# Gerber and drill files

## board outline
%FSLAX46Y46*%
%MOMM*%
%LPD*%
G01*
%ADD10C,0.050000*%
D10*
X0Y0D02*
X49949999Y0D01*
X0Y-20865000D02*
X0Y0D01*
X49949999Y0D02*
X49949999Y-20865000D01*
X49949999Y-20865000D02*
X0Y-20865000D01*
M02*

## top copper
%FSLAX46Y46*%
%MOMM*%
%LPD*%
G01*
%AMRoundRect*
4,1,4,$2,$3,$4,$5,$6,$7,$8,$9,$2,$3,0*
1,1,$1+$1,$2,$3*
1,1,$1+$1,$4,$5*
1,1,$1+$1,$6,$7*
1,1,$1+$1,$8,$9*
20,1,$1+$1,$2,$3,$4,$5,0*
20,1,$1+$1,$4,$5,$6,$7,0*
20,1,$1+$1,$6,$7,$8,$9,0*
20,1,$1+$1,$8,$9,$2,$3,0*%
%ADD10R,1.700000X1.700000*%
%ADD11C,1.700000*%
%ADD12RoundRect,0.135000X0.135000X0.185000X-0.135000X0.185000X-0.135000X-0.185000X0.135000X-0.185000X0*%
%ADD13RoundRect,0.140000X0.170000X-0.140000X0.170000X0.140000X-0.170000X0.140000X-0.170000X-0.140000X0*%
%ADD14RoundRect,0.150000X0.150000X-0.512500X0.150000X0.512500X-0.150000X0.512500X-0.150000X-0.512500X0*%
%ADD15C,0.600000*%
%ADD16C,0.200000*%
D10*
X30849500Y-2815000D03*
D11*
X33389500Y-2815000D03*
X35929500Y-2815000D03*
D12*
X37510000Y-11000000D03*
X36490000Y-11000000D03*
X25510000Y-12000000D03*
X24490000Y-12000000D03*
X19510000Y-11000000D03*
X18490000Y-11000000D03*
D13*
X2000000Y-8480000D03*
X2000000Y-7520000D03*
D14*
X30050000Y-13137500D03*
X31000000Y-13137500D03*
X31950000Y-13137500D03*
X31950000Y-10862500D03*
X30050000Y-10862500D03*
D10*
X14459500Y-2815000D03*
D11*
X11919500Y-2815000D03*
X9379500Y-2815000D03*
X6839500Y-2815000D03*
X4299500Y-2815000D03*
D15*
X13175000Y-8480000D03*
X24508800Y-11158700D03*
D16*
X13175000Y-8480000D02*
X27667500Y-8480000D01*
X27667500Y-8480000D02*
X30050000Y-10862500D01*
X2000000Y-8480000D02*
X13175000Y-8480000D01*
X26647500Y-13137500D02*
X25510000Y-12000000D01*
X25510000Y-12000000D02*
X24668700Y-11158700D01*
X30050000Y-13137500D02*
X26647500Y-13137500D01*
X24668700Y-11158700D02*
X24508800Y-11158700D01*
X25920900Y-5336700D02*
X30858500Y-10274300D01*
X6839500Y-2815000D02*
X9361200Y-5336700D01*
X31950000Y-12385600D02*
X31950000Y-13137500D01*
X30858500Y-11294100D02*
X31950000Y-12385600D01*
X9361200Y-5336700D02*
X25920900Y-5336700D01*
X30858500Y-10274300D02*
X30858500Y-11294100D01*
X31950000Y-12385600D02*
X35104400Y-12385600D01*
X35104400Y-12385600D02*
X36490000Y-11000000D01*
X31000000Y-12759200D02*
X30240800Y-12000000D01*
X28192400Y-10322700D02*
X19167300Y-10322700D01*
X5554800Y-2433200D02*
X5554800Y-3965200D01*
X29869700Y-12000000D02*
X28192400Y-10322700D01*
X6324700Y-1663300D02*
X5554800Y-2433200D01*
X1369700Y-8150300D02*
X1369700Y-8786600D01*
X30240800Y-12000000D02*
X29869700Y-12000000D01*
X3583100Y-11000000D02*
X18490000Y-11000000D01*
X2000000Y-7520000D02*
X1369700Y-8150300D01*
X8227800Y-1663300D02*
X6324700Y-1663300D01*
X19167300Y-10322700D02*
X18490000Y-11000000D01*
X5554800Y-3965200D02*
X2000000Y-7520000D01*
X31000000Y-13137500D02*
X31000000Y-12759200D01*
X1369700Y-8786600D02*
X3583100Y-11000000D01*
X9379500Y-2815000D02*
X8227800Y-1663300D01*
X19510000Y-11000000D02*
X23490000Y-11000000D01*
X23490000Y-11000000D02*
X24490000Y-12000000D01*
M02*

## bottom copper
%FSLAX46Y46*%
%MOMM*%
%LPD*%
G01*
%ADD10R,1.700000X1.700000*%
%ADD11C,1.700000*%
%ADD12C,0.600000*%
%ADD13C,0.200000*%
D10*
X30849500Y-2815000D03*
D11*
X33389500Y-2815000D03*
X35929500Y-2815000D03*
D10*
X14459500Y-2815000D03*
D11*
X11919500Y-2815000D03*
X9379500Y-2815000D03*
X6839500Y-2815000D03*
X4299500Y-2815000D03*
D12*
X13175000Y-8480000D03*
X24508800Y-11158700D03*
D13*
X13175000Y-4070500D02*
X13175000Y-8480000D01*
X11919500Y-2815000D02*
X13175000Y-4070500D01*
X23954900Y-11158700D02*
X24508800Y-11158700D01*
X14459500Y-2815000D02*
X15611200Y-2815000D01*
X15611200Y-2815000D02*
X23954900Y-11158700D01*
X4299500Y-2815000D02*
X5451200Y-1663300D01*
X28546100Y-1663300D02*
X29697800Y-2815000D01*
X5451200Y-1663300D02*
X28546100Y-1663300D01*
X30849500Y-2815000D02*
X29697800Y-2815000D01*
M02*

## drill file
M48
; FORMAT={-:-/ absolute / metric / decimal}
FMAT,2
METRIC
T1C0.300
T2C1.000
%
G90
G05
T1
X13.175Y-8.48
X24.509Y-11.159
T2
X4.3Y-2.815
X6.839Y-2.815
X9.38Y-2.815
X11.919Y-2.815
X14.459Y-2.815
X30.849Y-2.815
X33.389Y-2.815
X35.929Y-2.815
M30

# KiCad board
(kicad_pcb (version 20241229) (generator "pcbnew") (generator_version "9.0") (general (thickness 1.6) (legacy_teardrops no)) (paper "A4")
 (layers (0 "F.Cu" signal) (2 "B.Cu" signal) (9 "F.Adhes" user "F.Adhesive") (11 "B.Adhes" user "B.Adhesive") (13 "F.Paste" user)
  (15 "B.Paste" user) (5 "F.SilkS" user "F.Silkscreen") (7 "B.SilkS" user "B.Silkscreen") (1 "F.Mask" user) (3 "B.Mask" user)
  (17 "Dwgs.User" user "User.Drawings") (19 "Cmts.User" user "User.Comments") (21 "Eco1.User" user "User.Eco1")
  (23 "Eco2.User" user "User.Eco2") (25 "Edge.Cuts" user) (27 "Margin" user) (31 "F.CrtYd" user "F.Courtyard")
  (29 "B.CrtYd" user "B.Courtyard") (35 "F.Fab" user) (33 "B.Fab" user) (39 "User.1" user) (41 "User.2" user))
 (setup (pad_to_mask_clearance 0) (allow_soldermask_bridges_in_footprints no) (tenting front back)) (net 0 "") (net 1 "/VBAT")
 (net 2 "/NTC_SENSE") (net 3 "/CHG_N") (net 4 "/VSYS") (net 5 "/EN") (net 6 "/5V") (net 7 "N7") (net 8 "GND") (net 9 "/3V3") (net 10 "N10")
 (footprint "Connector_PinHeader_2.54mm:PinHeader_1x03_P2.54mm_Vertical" (layer "F.Cu") (at 30.8495 2.815 90)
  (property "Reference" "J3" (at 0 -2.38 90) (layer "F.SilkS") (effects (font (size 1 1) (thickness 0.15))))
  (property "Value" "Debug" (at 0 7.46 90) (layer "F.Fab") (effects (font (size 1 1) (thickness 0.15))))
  (pad "1" thru_hole rect (at 0 0 90) (size 1.7 1.7) (drill 1) (layers "*.Cu" "*.Mask") (remove_unused_layers no) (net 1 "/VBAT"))
  (pad "2" thru_hole circle (at 0 2.54 90) (size 1.7 1.7) (drill 1) (layers "*.Cu" "*.Mask") (remove_unused_layers no) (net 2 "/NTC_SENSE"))
  (pad "3" thru_hole circle (at 0 5.08 90) (size 1.7 1.7) (drill 1) (layers "*.Cu" "*.Mask") (remove_unused_layers no) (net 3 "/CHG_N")))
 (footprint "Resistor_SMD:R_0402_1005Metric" (layer "F.Cu") (at 37 11 180)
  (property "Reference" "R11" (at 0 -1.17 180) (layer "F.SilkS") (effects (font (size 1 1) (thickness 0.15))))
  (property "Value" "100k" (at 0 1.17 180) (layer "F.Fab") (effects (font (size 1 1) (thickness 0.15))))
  (pad "1" smd roundrect (at -0.51 0 180) (size 0.54 0.64) (layers "F.Cu" "F.Mask" "F.Paste") (roundrect_rratio 0.25) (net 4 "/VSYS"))
  (pad "2" smd roundrect (at 0.51 0 180) (size 0.54 0.64) (layers "F.Cu" "F.Mask" "F.Paste") (roundrect_rratio 0.25) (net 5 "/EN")))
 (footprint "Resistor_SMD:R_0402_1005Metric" (layer "F.Cu") (at 25 12 180)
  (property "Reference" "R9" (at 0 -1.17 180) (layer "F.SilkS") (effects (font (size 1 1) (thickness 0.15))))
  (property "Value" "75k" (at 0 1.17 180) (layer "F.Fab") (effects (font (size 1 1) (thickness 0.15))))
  (pad "1" smd roundrect (at -0.51 0 180) (size 0.54 0.64) (layers "F.Cu" "F.Mask" "F.Paste") (roundrect_rratio 0.25) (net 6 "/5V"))
  (pad "2" smd roundrect (at 0.51 0 180) (size 0.54 0.64) (layers "F.Cu" "F.Mask" "F.Paste") (roundrect_rratio 0.25) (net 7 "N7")))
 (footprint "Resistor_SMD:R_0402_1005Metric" (layer "F.Cu") (at 19 11 180)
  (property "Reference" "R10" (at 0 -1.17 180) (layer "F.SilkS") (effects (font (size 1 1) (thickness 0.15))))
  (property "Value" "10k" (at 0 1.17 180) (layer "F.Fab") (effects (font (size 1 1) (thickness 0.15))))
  (pad "1" smd roundrect (at -0.51 0 180) (size 0.54 0.64) (layers "F.Cu" "F.Mask" "F.Paste") (roundrect_rratio 0.25) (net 7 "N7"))
  (pad "2" smd roundrect (at 0.51 0 180) (size 0.54 0.64) (layers "F.Cu" "F.Mask" "F.Paste") (roundrect_rratio 0.25) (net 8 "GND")))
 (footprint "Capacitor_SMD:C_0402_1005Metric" (layer "F.Cu") (at 2 8 90)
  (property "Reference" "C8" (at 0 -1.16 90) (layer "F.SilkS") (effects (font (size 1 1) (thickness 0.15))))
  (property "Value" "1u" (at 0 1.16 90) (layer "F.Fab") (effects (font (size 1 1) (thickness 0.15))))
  (pad "1" smd roundrect (at -0.48 0 90) (size 0.56 0.62) (layers "F.Cu" "F.Mask" "F.Paste") (roundrect_rratio 0.25) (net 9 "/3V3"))
  (pad "2" smd roundrect (at 0.48 0 90) (size 0.56 0.62) (layers "F.Cu" "F.Mask" "F.Paste") (roundrect_rratio 0.25) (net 8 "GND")))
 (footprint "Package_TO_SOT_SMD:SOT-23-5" (layer "F.Cu") (at 31 12 90)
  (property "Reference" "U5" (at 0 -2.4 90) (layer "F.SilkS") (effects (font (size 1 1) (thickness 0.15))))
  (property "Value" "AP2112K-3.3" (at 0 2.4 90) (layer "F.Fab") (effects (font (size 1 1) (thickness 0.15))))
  (pad "1" smd roundrect (at -1.1375 -0.95 90) (size 1.325 0.6) (layers "F.Cu" "F.Mask" "F.Paste") (roundrect_rratio 0.25) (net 6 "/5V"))
  (pad "2" smd roundrect (at -1.1375 0 90) (size 1.325 0.6) (layers "F.Cu" "F.Mask" "F.Paste") (roundrect_rratio 0.25) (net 8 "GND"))
  (pad "3" smd roundrect (at -1.1375 0.95 90) (size 1.325 0.6) (layers "F.Cu" "F.Mask" "F.Paste") (roundrect_rratio 0.25) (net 5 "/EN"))
  (pad "4" smd roundrect (at 1.1375 0.95 90) (size 1.325 0.6) (layers "F.Cu" "F.Mask" "F.Paste") (roundrect_rratio 0.25) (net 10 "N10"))
  (pad "5" smd roundrect (at 1.1375 -0.95 90) (size 1.325 0.6) (layers "F.Cu" "F.Mask" "F.Paste") (roundrect_rratio 0.25) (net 9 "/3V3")))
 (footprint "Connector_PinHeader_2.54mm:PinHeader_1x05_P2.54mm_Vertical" (layer "B.Cu") (at 14.4595 2.815 90)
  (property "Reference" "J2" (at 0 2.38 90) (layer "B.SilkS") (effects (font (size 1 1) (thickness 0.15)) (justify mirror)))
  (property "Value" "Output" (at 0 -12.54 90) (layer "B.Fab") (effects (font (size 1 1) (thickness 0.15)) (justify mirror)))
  (pad "1" thru_hole rect (at 0 0 90) (size 1.7 1.7) (drill 1) (layers "*.Cu" "*.Mask") (remove_unused_layers no) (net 6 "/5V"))
  (pad "2" thru_hole circle (at 0 -2.54 90) (size 1.7 1.7) (drill 1) (layers "*.Cu" "*.Mask") (remove_unused_layers no) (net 9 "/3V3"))
  (pad "3" thru_hole circle (at 0 -5.08 90) (size 1.7 1.7) (drill 1) (layers "*.Cu" "*.Mask") (remove_unused_layers no) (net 8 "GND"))
  (pad "4" thru_hole circle (at 0 -7.62 90) (size 1.7 1.7) (drill 1) (layers "*.Cu" "*.Mask") (remove_unused_layers no) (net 5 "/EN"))
  (pad "5" thru_hole circle (at 0 -10.16 90) (size 1.7 1.7) (drill 1) (layers "*.Cu" "*.Mask") (remove_unused_layers no) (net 1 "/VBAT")))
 (gr_line (start 0 0) (end 49.949999 0) (stroke (width 0.05) (type default)) (layer "Edge.Cuts"))
 (gr_line (start 0 20.865) (end 0 0) (stroke (width 0.05) (type default)) (layer "Edge.Cuts"))
 (gr_line (start 49.949999 0) (end 49.949999 20.865) (stroke (width 0.05) (type default)) (layer "Edge.Cuts"))
 (gr_line (start 49.949999 20.865) (end 0 20.865) (stroke (width 0.05) (type default)) (layer "Edge.Cuts"))
 (segment (start 13.175 8.48) (end 27.6675 8.48) (width 0.2) (layer "F.Cu") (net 9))
 (segment (start 27.6675 8.48) (end 30.05 10.8625) (width 0.2) (layer "F.Cu") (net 9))
 (segment (start 2 8.48) (end 13.175 8.48) (width 0.2) (layer "F.Cu") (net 9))
 (via (at 13.175 8.48) (size 0.6) (drill 0.3) (layers "F.Cu" "B.Cu") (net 9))
 (segment (start 13.175 4.0705) (end 13.175 8.48) (width 0.2) (layer "B.Cu") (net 9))
 (segment (start 11.9195 2.815) (end 13.175 4.0705) (width 0.2) (layer "B.Cu") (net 9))
 (segment (start 26.6475 13.1375) (end 25.51 12) (width 0.2) (layer "F.Cu") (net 6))
 (segment (start 25.51 12) (end 24.6687 11.1587) (width 0.2) (layer "F.Cu") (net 6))
 (segment (start 30.05 13.1375) (end 26.6475 13.1375) (width 0.2) (layer "F.Cu") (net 6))
 (segment (start 24.6687 11.1587) (end 24.5088 11.1587) (width 0.2) (layer "F.Cu") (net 6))
 (via (at 24.5088 11.1587) (size 0.6) (drill 0.3) (layers "F.Cu" "B.Cu") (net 6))
 (segment (start 23.9549 11.1587) (end 24.5088 11.1587) (width 0.2) (layer "B.Cu") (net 6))
 (segment (start 14.4595 2.815) (end 15.6112 2.815) (width 0.2) (layer "B.Cu") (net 6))
 (segment (start 15.6112 2.815) (end 23.9549 11.1587) (width 0.2) (layer "B.Cu") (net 6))
 (segment (start 25.9209 5.3367) (end 30.8585 10.2743) (width 0.2) (layer "F.Cu") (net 5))
 (segment (start 6.8395 2.815) (end 9.3612 5.3367) (width 0.2) (layer "F.Cu") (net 5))
 (segment (start 31.95 12.3856) (end 31.95 13.1375) (width 0.2) (layer "F.Cu") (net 5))
 (segment (start 30.8585 11.2941) (end 31.95 12.3856) (width 0.2) (layer "F.Cu") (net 5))
 (segment (start 9.3612 5.3367) (end 25.9209 5.3367) (width 0.2) (layer "F.Cu") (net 5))
 (segment (start 30.8585 10.2743) (end 30.8585 11.2941) (width 0.2) (layer "F.Cu") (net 5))
 (segment (start 31.95 12.3856) (end 35.1044 12.3856) (width 0.2) (layer "F.Cu") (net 5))
 (segment (start 35.1044 12.3856) (end 36.49 11) (width 0.2) (layer "F.Cu") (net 5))
 (segment (start 4.2995 2.815) (end 5.4512 1.6633) (width 0.2) (layer "B.Cu") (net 1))
 (segment (start 28.5461 1.6633) (end 29.6978 2.815) (width 0.2) (layer "B.Cu") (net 1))
 (segment (start 5.4512 1.6633) (end 28.5461 1.6633) (width 0.2) (layer "B.Cu") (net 1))
 (segment (start 30.8495 2.815) (end 29.6978 2.815) (width 0.2) (layer "B.Cu") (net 1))
 (segment (start 31 12.7592) (end 30.2408 12) (width 0.2) (layer "F.Cu") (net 8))
 (segment (start 28.1924 10.3227) (end 19.1673 10.3227) (width 0.2) (layer "F.Cu") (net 8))
 (segment (start 5.5548 2.4332) (end 5.5548 3.9652) (width 0.2) (layer "F.Cu") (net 8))
 (segment (start 29.8697 12) (end 28.1924 10.3227) (width 0.2) (layer "F.Cu") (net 8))
 (segment (start 6.3247 1.6633) (end 5.5548 2.4332) (width 0.2) (layer "F.Cu") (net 8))
 (segment (start 1.3697 8.1503) (end 1.3697 8.7866) (width 0.2) (layer "F.Cu") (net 8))
 (segment (start 30.2408 12) (end 29.8697 12) (width 0.2) (layer "F.Cu") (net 8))
 (segment (start 3.5831 11) (end 18.49 11) (width 0.2) (layer "F.Cu") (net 8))
 (segment (start 2 7.52) (end 1.3697 8.1503) (width 0.2) (layer "F.Cu") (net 8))
 (segment (start 8.2278 1.6633) (end 6.3247 1.6633) (width 0.2) (layer "F.Cu") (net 8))
 (segment (start 19.1673 10.3227) (end 18.49 11) (width 0.2) (layer "F.Cu") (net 8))
 (segment (start 5.5548 3.9652) (end 2 7.52) (width 0.2) (layer "F.Cu") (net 8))
 (segment (start 31 13.1375) (end 31 12.7592) (width 0.2) (layer "F.Cu") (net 8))
 (segment (start 1.3697 8.7866) (end 3.5831 11) (width 0.2) (layer "F.Cu") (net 8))
 (segment (start 9.3795 2.815) (end 8.2278 1.6633) (width 0.2) (layer "F.Cu") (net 8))
 (segment (start 19.51 11) (end 23.49 11) (width 0.2) (layer "F.Cu") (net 7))
 (segment (start 23.49 11) (end 24.49 12) (width 0.2) (layer "F.Cu") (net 7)))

